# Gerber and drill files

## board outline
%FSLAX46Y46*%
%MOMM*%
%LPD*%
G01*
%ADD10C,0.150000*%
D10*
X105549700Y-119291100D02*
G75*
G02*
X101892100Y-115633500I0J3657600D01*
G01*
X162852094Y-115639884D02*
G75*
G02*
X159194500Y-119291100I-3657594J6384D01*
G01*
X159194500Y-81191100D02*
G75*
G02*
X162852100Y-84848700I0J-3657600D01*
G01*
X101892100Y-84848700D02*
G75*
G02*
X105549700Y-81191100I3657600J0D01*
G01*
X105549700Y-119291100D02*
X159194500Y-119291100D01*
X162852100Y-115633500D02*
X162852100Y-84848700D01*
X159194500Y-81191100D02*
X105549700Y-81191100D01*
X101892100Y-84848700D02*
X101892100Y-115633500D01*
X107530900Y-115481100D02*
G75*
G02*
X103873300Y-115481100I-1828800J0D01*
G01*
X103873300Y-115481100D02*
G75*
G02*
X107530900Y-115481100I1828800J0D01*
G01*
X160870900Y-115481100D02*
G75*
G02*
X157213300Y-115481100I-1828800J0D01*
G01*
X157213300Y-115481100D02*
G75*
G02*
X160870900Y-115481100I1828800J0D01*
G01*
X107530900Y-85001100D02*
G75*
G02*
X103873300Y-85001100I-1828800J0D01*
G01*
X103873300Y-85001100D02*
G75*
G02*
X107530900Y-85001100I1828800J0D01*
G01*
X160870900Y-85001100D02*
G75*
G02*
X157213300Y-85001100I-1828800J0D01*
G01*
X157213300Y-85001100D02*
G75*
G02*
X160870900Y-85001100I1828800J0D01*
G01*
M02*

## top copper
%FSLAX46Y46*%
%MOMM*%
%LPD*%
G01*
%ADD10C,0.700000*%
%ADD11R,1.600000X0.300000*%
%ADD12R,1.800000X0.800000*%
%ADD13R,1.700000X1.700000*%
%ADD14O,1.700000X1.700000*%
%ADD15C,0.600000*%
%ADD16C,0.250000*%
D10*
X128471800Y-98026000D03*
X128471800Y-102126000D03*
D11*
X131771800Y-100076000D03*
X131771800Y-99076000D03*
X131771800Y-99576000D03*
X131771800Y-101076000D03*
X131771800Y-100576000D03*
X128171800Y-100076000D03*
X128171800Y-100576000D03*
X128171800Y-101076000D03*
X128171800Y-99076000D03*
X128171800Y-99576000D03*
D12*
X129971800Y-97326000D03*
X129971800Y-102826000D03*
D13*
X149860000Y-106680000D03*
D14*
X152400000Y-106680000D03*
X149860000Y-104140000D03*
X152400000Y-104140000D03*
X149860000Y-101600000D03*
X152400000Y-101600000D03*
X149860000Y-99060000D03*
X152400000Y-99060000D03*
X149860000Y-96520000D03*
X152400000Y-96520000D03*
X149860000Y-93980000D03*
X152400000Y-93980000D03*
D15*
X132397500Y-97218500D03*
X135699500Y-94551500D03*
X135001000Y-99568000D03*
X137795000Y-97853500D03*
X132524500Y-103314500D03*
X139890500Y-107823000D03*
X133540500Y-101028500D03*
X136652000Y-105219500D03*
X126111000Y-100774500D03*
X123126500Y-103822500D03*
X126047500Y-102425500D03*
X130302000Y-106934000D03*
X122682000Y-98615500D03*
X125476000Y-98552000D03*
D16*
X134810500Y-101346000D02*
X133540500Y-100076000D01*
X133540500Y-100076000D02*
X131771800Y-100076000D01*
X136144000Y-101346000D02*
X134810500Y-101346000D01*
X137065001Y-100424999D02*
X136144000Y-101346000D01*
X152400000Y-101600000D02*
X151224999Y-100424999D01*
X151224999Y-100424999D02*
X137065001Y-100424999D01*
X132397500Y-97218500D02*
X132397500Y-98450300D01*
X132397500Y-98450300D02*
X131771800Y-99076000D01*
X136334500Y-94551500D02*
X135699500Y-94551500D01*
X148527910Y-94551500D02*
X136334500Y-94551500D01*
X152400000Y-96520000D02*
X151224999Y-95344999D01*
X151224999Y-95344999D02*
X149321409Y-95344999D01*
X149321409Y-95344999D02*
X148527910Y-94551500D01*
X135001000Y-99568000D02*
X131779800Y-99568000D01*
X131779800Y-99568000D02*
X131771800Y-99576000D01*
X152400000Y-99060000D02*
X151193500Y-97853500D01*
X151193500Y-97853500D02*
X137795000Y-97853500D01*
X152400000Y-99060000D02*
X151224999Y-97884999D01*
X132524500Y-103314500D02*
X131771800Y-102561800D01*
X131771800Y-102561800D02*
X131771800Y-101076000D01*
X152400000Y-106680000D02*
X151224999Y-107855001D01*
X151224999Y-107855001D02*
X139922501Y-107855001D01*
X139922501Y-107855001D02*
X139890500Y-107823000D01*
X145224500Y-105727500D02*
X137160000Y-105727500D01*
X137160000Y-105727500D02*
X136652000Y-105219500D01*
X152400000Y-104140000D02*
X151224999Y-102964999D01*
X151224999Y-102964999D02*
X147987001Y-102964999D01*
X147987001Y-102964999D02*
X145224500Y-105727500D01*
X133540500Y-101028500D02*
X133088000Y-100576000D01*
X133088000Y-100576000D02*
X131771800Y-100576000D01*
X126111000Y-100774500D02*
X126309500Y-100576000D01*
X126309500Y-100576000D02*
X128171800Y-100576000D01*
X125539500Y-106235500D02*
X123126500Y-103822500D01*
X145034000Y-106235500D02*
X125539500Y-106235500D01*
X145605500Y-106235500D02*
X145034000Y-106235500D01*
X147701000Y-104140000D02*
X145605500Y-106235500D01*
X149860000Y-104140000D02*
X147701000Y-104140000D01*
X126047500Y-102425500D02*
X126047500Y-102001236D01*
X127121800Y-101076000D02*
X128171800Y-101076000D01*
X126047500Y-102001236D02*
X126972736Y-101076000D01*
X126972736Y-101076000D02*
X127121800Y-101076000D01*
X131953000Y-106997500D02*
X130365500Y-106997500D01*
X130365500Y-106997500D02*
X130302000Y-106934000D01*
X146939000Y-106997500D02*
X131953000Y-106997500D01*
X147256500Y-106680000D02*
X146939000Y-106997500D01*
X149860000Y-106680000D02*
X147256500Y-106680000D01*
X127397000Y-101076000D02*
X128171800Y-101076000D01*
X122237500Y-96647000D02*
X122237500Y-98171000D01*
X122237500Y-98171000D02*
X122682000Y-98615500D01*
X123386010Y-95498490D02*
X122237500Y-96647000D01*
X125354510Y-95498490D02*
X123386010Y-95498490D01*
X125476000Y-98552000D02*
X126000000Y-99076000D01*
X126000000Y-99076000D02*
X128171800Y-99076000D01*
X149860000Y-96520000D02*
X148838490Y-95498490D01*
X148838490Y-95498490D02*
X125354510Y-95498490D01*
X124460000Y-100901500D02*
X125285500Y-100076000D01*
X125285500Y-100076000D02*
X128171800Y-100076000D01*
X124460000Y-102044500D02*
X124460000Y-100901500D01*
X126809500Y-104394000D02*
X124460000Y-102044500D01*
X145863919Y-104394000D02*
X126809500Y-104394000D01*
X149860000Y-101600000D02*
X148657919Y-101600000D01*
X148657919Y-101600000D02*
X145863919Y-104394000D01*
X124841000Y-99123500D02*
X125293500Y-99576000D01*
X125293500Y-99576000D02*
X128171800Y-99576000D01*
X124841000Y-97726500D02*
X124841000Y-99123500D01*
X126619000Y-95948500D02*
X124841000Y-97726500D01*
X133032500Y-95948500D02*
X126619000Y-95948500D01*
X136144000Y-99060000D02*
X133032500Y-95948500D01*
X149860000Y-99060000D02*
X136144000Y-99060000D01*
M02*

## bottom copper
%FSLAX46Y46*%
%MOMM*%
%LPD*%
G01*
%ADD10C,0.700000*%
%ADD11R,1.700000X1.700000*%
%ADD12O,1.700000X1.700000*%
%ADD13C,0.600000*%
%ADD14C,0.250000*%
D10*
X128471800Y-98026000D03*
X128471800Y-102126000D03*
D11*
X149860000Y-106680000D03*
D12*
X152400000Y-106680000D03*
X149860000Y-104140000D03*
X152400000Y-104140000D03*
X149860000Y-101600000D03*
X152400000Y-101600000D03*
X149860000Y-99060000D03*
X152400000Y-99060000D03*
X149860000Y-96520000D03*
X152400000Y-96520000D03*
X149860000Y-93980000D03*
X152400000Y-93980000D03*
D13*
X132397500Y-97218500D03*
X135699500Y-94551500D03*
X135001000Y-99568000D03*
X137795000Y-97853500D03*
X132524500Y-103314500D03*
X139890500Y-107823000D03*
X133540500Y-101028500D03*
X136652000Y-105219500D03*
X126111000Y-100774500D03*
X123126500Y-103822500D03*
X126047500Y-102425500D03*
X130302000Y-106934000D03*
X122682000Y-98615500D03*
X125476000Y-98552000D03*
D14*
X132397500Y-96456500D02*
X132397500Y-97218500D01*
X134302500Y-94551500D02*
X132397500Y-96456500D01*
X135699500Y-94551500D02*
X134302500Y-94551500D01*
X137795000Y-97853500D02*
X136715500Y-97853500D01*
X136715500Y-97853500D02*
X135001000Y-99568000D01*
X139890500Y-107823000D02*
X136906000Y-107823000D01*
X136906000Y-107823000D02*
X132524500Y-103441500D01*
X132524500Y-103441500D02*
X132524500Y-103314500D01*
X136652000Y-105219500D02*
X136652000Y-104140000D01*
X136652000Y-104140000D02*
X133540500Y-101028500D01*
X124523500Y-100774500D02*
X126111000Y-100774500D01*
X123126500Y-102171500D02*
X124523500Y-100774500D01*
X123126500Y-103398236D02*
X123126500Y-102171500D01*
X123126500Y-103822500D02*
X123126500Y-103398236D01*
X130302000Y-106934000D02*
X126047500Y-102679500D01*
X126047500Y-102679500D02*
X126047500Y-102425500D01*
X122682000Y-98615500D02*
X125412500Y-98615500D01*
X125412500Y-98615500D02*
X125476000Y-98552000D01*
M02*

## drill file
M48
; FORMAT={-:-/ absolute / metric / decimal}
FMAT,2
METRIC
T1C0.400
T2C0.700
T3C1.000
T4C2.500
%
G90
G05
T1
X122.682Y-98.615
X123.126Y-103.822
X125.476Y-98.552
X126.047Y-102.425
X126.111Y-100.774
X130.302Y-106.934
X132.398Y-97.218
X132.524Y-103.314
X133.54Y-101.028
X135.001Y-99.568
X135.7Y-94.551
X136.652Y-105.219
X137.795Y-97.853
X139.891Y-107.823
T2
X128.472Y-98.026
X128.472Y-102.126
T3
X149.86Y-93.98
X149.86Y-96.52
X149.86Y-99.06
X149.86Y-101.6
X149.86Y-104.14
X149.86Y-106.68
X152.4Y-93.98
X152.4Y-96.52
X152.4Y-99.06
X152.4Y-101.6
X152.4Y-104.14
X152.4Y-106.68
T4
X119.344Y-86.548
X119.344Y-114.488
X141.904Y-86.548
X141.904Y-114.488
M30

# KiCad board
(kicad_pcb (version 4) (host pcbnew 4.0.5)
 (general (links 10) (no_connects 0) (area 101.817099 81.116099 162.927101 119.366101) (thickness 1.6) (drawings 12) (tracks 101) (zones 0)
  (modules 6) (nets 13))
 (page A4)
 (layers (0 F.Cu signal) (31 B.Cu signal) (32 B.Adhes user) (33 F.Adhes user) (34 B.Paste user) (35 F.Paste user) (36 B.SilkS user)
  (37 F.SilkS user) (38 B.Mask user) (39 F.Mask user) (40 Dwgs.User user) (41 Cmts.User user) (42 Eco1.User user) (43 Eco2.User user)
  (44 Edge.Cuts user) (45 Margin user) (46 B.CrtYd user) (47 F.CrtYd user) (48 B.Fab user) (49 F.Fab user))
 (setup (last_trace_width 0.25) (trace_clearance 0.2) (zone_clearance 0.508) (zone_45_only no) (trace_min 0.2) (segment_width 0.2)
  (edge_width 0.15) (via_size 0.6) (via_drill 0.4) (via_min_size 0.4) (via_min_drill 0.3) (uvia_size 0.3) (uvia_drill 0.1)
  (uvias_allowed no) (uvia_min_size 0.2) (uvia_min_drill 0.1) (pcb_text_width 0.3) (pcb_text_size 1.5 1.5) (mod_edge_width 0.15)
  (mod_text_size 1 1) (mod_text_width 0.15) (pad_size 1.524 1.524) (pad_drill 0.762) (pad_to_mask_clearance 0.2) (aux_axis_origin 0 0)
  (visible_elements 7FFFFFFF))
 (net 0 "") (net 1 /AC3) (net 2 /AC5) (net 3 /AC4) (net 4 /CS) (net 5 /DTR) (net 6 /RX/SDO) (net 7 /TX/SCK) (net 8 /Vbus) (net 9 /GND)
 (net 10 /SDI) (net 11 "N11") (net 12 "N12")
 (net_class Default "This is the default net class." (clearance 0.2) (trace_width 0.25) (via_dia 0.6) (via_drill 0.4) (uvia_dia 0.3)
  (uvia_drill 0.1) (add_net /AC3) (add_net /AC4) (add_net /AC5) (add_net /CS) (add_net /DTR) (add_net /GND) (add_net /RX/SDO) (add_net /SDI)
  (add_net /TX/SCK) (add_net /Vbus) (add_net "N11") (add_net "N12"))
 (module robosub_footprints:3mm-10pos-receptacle (layer F.Cu) (at 129.9718 100.076 90)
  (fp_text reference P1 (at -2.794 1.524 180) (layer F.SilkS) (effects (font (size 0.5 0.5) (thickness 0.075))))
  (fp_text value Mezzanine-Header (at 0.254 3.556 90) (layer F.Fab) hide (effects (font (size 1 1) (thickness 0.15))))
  (pad "" thru_hole circle (at 2.05 -1.5 90) (size 0.7 0.7) (drill 0.7) (layers *.Cu *.Mask))
  (pad "" thru_hole circle (at -2.05 -1.5 90) (size 0.7 0.7) (drill 0.7) (layers *.Cu *.Mask))
  (pad 6 smd rect (at 0 1.8 90) (size 0.3 1.6) (layers F.Cu F.Paste F.Mask) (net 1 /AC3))
  (pad 10 smd rect (at 1 1.8 90) (size 0.3 1.6) (layers F.Cu F.Paste F.Mask) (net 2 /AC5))
  (pad 8 smd rect (at 0.5 1.8 90) (size 0.3 1.6) (layers F.Cu F.Paste F.Mask) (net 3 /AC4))
  (pad 2 smd rect (at -1 1.8 90) (size 0.3 1.6) (layers F.Cu F.Paste F.Mask) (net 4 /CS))
  (pad 4 smd rect (at -0.5 1.8 90) (size 0.3 1.6) (layers F.Cu F.Paste F.Mask) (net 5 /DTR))
  (pad 5 smd rect (at 0 -1.8 90) (size 0.3 1.6) (layers F.Cu F.Paste F.Mask) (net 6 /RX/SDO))
  (pad 3 smd rect (at -0.5 -1.8 90) (size 0.3 1.6) (layers F.Cu F.Paste F.Mask) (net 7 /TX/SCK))
  (pad 1 smd rect (at -1 -1.8 90) (size 0.3 1.6) (layers F.Cu F.Paste F.Mask) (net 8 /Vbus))
  (pad 9 smd rect (at 1 -1.8 90) (size 0.3 1.6) (layers F.Cu F.Paste F.Mask) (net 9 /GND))
  (pad 7 smd rect (at 0.5 -1.8 90) (size 0.3 1.6) (layers F.Cu F.Paste F.Mask) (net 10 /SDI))
  (pad "" smd rect (at 2.75 0 90) (size 0.8 1.8) (layers F.Cu F.Paste F.Mask))
  (pad "" smd rect (at -2.75 0 90) (size 0.8 1.8) (layers F.Cu F.Paste F.Mask)))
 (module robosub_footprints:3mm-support (layer F.Cu) (at 119.3442 86.548204)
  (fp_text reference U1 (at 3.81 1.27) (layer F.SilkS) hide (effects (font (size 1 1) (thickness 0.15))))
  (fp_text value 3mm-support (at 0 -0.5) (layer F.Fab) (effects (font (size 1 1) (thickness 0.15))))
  (pad "" np_thru_hole circle (at 0 0) (size 2.5 2.5) (drill 2.5) (layers *.Cu *.Mask)))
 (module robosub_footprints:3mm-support (layer F.Cu) (at 141.9042 86.548204)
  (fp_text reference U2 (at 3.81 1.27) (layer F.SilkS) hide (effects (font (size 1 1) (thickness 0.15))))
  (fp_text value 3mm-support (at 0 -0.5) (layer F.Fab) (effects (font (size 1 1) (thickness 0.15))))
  (pad "" np_thru_hole circle (at 0 0) (size 2.5 2.5) (drill 2.5) (layers *.Cu *.Mask)))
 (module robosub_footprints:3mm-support (layer F.Cu) (at 119.3442 114.488204)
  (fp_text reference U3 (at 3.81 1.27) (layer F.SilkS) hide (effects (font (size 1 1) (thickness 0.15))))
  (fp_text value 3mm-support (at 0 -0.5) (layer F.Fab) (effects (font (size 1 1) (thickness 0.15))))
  (pad "" np_thru_hole circle (at 0 0) (size 2.5 2.5) (drill 2.5) (layers *.Cu *.Mask)))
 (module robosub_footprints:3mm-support (layer F.Cu) (at 141.9042 114.488204)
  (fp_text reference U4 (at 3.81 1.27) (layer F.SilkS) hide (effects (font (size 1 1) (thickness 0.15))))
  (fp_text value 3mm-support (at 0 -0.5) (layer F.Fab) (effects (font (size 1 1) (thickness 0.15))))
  (pad "" np_thru_hole circle (at 0 0) (size 2.5 2.5) (drill 2.5) (layers *.Cu *.Mask)))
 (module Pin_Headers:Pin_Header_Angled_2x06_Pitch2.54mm (layer B.Cu) (at 149.86 106.68)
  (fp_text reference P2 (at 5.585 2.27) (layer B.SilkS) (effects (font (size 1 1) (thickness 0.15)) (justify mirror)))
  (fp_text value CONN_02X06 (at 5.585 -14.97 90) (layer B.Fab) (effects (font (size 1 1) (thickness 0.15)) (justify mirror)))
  (pad 1 thru_hole rect (at 0 0) (size 1.7 1.7) (drill 1) (layers *.Cu *.Mask) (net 8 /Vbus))
  (pad 2 thru_hole oval (at 2.54 0) (size 1.7 1.7) (drill 1) (layers *.Cu *.Mask) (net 4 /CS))
  (pad 3 thru_hole oval (at 0 -2.54) (size 1.7 1.7) (drill 1) (layers *.Cu *.Mask) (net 7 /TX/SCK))
  (pad 4 thru_hole oval (at 2.54 -2.54) (size 1.7 1.7) (drill 1) (layers *.Cu *.Mask) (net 5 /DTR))
  (pad 5 thru_hole oval (at 0 -5.08) (size 1.7 1.7) (drill 1) (layers *.Cu *.Mask) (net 6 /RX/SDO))
  (pad 6 thru_hole oval (at 2.54 -5.08) (size 1.7 1.7) (drill 1) (layers *.Cu *.Mask) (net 1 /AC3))
  (pad 7 thru_hole oval (at 0 -7.62) (size 1.7 1.7) (drill 1) (layers *.Cu *.Mask) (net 10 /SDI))
  (pad 8 thru_hole oval (at 2.54 -7.62) (size 1.7 1.7) (drill 1) (layers *.Cu *.Mask) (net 3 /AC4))
  (pad 9 thru_hole oval (at 0 -10.16) (size 1.7 1.7) (drill 1) (layers *.Cu *.Mask) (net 9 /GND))
  (pad 10 thru_hole oval (at 2.54 -10.16) (size 1.7 1.7) (drill 1) (layers *.Cu *.Mask) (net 2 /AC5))
  (pad 11 thru_hole oval (at 0 -12.7) (size 1.7 1.7) (drill 1) (layers *.Cu *.Mask) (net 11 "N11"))
  (pad 12 thru_hole oval (at 2.54 -12.7) (size 1.7 1.7) (drill 1) (layers *.Cu *.Mask) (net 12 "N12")))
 (gr_arc (start 105.5497 115.6335) (end 101.8921 115.6335) (angle -90) (layer Edge.Cuts) (width 0.15))
 (gr_arc (start 159.1945 115.6335) (end 159.1945 119.2911) (angle -89.9) (layer Edge.Cuts) (width 0.15))
 (gr_arc (start 159.1945 84.8487) (end 162.8521 84.8487) (angle -90) (layer Edge.Cuts) (width 0.15))
 (gr_arc (start 105.5497 84.8487) (end 105.5497 81.1911) (angle -90) (layer Edge.Cuts) (width 0.15))
 (gr_line (start 105.5497 119.2911) (end 159.1945 119.2911) (layer Edge.Cuts) (width 0.15))
 (gr_line (start 162.8521 115.6335) (end 162.8521 84.8487) (layer Edge.Cuts) (width 0.15))
 (gr_line (start 159.1945 81.1911) (end 105.5497 81.1911) (layer Edge.Cuts) (width 0.15))
 (gr_line (start 101.8921 84.8487) (end 101.8921 115.6335) (layer Edge.Cuts) (width 0.15))
 (gr_circle (center 105.7021 115.4811) (end 107.5309 115.4811) (layer Edge.Cuts) (width 0.15))
 (gr_circle (center 159.0421 115.4811) (end 160.8709 115.4811) (layer Edge.Cuts) (width 0.15))
 (gr_circle (center 105.7021 85.0011) (end 107.5309 85.0011) (layer Edge.Cuts) (width 0.15))
 (gr_circle (center 159.0421 85.0011) (end 160.8709 85.0011) (layer Edge.Cuts) (width 0.15))
 (segment (start 134.8105 101.346) (end 133.5405 100.076) (width 0.25) (layer F.Cu) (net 1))
 (segment (start 133.5405 100.076) (end 131.7718 100.076) (width 0.25) (layer F.Cu) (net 1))
 (segment (start 136.144 101.346) (end 134.8105 101.346) (width 0.25) (layer F.Cu) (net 1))
 (segment (start 137.065001 100.424999) (end 136.144 101.346) (width 0.25) (layer F.Cu) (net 1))
 (segment (start 152.4 101.6) (end 151.224999 100.424999) (width 0.25) (layer F.Cu) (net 1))
 (segment (start 151.224999 100.424999) (end 137.065001 100.424999) (width 0.25) (layer F.Cu) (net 1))
 (segment (start 132.3975 97.2185) (end 132.3975 98.4503) (width 0.25) (layer F.Cu) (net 2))
 (segment (start 132.3975 98.4503) (end 131.7718 99.076) (width 0.25) (layer F.Cu) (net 2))
 (segment (start 132.3975 96.4565) (end 132.3975 97.2185) (width 0.25) (layer B.Cu) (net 2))
 (via (at 132.3975 97.2185) (size 0.6) (drill 0.4) (layers F.Cu B.Cu) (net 2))
 (segment (start 134.3025 94.5515) (end 132.3975 96.4565) (width 0.25) (layer B.Cu) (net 2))
 (segment (start 135.6995 94.5515) (end 134.3025 94.5515) (width 0.25) (layer B.Cu) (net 2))
 (segment (start 136.3345 94.5515) (end 135.6995 94.5515) (width 0.25) (layer F.Cu) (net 2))
 (via (at 135.6995 94.5515) (size 0.6) (drill 0.4) (layers F.Cu B.Cu) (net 2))
 (segment (start 148.52791 94.5515) (end 136.3345 94.5515) (width 0.25) (layer F.Cu) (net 2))
 (segment (start 152.4 96.52) (end 151.224999 95.344999) (width 0.25) (layer F.Cu) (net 2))
 (segment (start 151.224999 95.344999) (end 149.321409 95.344999) (width 0.25) (layer F.Cu) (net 2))
 (segment (start 149.321409 95.344999) (end 148.52791 94.5515) (width 0.25) (layer F.Cu) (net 2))
 (segment (start 135.001 99.568) (end 131.7798 99.568) (width 0.25) (layer F.Cu) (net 3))
 (segment (start 131.7798 99.568) (end 131.7718 99.576) (width 0.25) (layer F.Cu) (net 3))
 (segment (start 137.795 97.8535) (end 136.7155 97.8535) (width 0.25) (layer B.Cu) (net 3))
 (segment (start 136.7155 97.8535) (end 135.001 99.568) (width 0.25) (layer B.Cu) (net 3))
 (via (at 135.001 99.568) (size 0.6) (drill 0.4) (layers F.Cu B.Cu) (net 3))
 (segment (start 152.4 99.06) (end 151.1935 97.8535) (width 0.25) (layer F.Cu) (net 3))
 (segment (start 151.1935 97.8535) (end 137.795 97.8535) (width 0.25) (layer F.Cu) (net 3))
 (via (at 137.795 97.8535) (size 0.6) (drill 0.4) (layers F.Cu B.Cu) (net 3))
 (segment (start 152.4 99.06) (end 151.224999 97.884999) (width 0.25) (layer F.Cu) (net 3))
 (segment (start 132.5245 103.3145) (end 131.7718 102.5618) (width 0.25) (layer F.Cu) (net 4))
 (segment (start 131.7718 102.5618) (end 131.7718 101.076) (width 0.25) (layer F.Cu) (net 4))
 (segment (start 139.8905 107.823) (end 136.906 107.823) (width 0.25) (layer B.Cu) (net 4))
 (segment (start 136.906 107.823) (end 132.5245 103.4415) (width 0.25) (layer B.Cu) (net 4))
 (segment (start 132.5245 103.4415) (end 132.5245 103.3145) (width 0.25) (layer B.Cu) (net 4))
 (via (at 132.5245 103.3145) (size 0.6) (drill 0.4) (layers F.Cu B.Cu) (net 4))
 (segment (start 152.4 106.68) (end 151.224999 107.855001) (width 0.25) (layer F.Cu) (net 4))
 (segment (start 151.224999 107.855001) (end 139.922501 107.855001) (width 0.25) (layer F.Cu) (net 4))
 (segment (start 139.922501 107.855001) (end 139.8905 107.823) (width 0.25) (layer F.Cu) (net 4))
 (via (at 139.8905 107.823) (size 0.6) (drill 0.4) (layers F.Cu B.Cu) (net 4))
 (segment (start 145.2245 105.7275) (end 137.16 105.7275) (width 0.25) (layer F.Cu) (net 5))
 (segment (start 137.16 105.7275) (end 136.652 105.2195) (width 0.25) (layer F.Cu) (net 5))
 (segment (start 152.4 104.14) (end 151.224999 102.964999) (width 0.25) (layer F.Cu) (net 5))
 (segment (start 151.224999 102.964999) (end 147.987001 102.964999) (width 0.25) (layer F.Cu) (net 5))
 (segment (start 147.987001 102.964999) (end 145.2245 105.7275) (width 0.25) (layer F.Cu) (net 5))
 (segment (start 133.5405 101.0285) (end 133.088 100.576) (width 0.25) (layer F.Cu) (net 5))
 (segment (start 133.088 100.576) (end 131.7718 100.576) (width 0.25) (layer F.Cu) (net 5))
 (segment (start 136.652 105.2195) (end 136.652 104.14) (width 0.25) (layer B.Cu) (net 5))
 (segment (start 136.652 104.14) (end 133.5405 101.0285) (width 0.25) (layer B.Cu) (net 5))
 (via (at 133.5405 101.0285) (size 0.6) (drill 0.4) (layers F.Cu B.Cu) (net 5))
 (via (at 136.652 105.2195) (size 0.6) (drill 0.4) (layers F.Cu B.Cu) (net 5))
 (segment (start 126.111 100.7745) (end 126.3095 100.576) (width 0.25) (layer F.Cu) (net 7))
 (segment (start 126.3095 100.576) (end 128.1718 100.576) (width 0.25) (layer F.Cu) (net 7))
 (segment (start 124.5235 100.7745) (end 126.111 100.7745) (width 0.25) (layer B.Cu) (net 7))
 (via (at 126.111 100.7745) (size 0.6) (drill 0.4) (layers F.Cu B.Cu) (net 7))
 (segment (start 123.1265 102.1715) (end 124.5235 100.7745) (width 0.25) (layer B.Cu) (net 7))
 (segment (start 123.1265 103.398236) (end 123.1265 102.1715) (width 0.25) (layer B.Cu) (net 7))
 (segment (start 123.1265 103.8225) (end 123.1265 103.398236) (width 0.25) (layer B.Cu) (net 7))
 (via (at 123.1265 103.8225) (size 0.6) (drill 0.4) (layers F.Cu B.Cu) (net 7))
 (segment (start 125.5395 106.2355) (end 123.1265 103.8225) (width 0.25) (layer F.Cu) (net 7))
 (segment (start 145.034 106.2355) (end 125.5395 106.2355) (width 0.25) (layer F.Cu) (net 7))
 (segment (start 145.6055 106.2355) (end 145.034 106.2355) (width 0.25) (layer F.Cu) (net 7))
 (segment (start 147.701 104.14) (end 145.6055 106.2355) (width 0.25) (layer F.Cu) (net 7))
 (segment (start 149.86 104.14) (end 147.701 104.14) (width 0.25) (layer F.Cu) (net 7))
 (segment (start 126.0475 102.4255) (end 126.0475 102.001236) (width 0.25) (layer F.Cu) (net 8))
 (segment (start 127.1218 101.076) (end 128.1718 101.076) (width 0.25) (layer F.Cu) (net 8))
 (segment (start 126.0475 102.001236) (end 126.972736 101.076) (width 0.25) (layer F.Cu) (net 8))
 (segment (start 126.972736 101.076) (end 127.1218 101.076) (width 0.25) (layer F.Cu) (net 8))
 (segment (start 130.302 106.934) (end 126.0475 102.6795) (width 0.25) (layer B.Cu) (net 8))
 (segment (start 126.0475 102.6795) (end 126.0475 102.4255) (width 0.25) (layer B.Cu) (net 8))
 (via (at 126.0475 102.4255) (size 0.6) (drill 0.4) (layers F.Cu B.Cu) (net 8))
 (segment (start 131.953 106.9975) (end 130.3655 106.9975) (width 0.25) (layer F.Cu) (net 8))
 (segment (start 130.3655 106.9975) (end 130.302 106.934) (width 0.25) (layer F.Cu) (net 8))
 (via (at 130.302 106.934) (size 0.6) (drill 0.4) (layers F.Cu B.Cu) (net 8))
 (segment (start 146.939 106.9975) (end 131.953 106.9975) (width 0.25) (layer F.Cu) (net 8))
 (segment (start 147.2565 106.68) (end 146.939 106.9975) (width 0.25) (layer F.Cu) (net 8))
 (segment (start 149.86 106.68) (end 147.2565 106.68) (width 0.25) (layer F.Cu) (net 8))
 (segment (start 127.397 101.076) (end 128.1718 101.076) (width 0.25) (layer F.Cu) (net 8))
 (segment (start 122.682 98.6155) (end 125.4125 98.6155) (width 0.25) (layer B.Cu) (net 9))
 (segment (start 125.4125 98.6155) (end 125.476 98.552) (width 0.25) (layer B.Cu) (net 9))
 (segment (start 122.2375 96.647) (end 122.2375 98.171) (width 0.25) (layer F.Cu) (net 9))
 (segment (start 122.2375 98.171) (end 122.682 98.6155) (width 0.25) (layer F.Cu) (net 9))
 (via (at 122.682 98.6155) (size 0.6) (drill 0.4) (layers F.Cu B.Cu) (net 9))
 (segment (start 123.38601 95.49849) (end 122.2375 96.647) (width 0.25) (layer F.Cu) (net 9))
 (segment (start 125.35451 95.49849) (end 123.38601 95.49849) (width 0.25) (layer F.Cu) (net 9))
 (segment (start 125.476 98.552) (end 126 99.076) (width 0.25) (layer F.Cu) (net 9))
 (segment (start 126 99.076) (end 128.1718 99.076) (width 0.25) (layer F.Cu) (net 9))
 (via (at 125.476 98.552) (size 0.6) (drill 0.4) (layers F.Cu B.Cu) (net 9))
 (segment (start 149.86 96.52) (end 148.83849 95.49849) (width 0.25) (layer F.Cu) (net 9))
 (segment (start 148.83849 95.49849) (end 125.35451 95.49849) (width 0.25) (layer F.Cu) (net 9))
 (segment (start 124.46 100.9015) (end 125.2855 100.076) (width 0.25) (layer F.Cu) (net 6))
 (segment (start 125.2855 100.076) (end 128.1718 100.076) (width 0.25) (layer F.Cu) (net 6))
 (segment (start 124.46 102.0445) (end 124.46 100.9015) (width 0.25) (layer F.Cu) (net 6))
 (segment (start 126.8095 104.394) (end 124.46 102.0445) (width 0.25) (layer F.Cu) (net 6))
 (segment (start 145.863919 104.394) (end 126.8095 104.394) (width 0.25) (layer F.Cu) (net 6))
 (segment (start 149.86 101.6) (end 148.657919 101.6) (width 0.25) (layer F.Cu) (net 6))
 (segment (start 148.657919 101.6) (end 145.863919 104.394) (width 0.25) (layer F.Cu) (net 6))
 (segment (start 124.841 99.1235) (end 125.2935 99.576) (width 0.25) (layer F.Cu) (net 10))
 (segment (start 125.2935 99.576) (end 128.1718 99.576) (width 0.25) (layer F.Cu) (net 10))
 (segment (start 124.841 97.7265) (end 124.841 99.1235) (width 0.25) (layer F.Cu) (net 10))
 (segment (start 126.619 95.9485) (end 124.841 97.7265) (width 0.25) (layer F.Cu) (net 10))
 (segment (start 133.0325 95.9485) (end 126.619 95.9485) (width 0.25) (layer F.Cu) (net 10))
 (segment (start 136.144 99.06) (end 133.0325 95.9485) (width 0.25) (layer F.Cu) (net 10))
 (segment (start 149.86 99.06) (end 136.144 99.06) (width 0.25) (layer F.Cu) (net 10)))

